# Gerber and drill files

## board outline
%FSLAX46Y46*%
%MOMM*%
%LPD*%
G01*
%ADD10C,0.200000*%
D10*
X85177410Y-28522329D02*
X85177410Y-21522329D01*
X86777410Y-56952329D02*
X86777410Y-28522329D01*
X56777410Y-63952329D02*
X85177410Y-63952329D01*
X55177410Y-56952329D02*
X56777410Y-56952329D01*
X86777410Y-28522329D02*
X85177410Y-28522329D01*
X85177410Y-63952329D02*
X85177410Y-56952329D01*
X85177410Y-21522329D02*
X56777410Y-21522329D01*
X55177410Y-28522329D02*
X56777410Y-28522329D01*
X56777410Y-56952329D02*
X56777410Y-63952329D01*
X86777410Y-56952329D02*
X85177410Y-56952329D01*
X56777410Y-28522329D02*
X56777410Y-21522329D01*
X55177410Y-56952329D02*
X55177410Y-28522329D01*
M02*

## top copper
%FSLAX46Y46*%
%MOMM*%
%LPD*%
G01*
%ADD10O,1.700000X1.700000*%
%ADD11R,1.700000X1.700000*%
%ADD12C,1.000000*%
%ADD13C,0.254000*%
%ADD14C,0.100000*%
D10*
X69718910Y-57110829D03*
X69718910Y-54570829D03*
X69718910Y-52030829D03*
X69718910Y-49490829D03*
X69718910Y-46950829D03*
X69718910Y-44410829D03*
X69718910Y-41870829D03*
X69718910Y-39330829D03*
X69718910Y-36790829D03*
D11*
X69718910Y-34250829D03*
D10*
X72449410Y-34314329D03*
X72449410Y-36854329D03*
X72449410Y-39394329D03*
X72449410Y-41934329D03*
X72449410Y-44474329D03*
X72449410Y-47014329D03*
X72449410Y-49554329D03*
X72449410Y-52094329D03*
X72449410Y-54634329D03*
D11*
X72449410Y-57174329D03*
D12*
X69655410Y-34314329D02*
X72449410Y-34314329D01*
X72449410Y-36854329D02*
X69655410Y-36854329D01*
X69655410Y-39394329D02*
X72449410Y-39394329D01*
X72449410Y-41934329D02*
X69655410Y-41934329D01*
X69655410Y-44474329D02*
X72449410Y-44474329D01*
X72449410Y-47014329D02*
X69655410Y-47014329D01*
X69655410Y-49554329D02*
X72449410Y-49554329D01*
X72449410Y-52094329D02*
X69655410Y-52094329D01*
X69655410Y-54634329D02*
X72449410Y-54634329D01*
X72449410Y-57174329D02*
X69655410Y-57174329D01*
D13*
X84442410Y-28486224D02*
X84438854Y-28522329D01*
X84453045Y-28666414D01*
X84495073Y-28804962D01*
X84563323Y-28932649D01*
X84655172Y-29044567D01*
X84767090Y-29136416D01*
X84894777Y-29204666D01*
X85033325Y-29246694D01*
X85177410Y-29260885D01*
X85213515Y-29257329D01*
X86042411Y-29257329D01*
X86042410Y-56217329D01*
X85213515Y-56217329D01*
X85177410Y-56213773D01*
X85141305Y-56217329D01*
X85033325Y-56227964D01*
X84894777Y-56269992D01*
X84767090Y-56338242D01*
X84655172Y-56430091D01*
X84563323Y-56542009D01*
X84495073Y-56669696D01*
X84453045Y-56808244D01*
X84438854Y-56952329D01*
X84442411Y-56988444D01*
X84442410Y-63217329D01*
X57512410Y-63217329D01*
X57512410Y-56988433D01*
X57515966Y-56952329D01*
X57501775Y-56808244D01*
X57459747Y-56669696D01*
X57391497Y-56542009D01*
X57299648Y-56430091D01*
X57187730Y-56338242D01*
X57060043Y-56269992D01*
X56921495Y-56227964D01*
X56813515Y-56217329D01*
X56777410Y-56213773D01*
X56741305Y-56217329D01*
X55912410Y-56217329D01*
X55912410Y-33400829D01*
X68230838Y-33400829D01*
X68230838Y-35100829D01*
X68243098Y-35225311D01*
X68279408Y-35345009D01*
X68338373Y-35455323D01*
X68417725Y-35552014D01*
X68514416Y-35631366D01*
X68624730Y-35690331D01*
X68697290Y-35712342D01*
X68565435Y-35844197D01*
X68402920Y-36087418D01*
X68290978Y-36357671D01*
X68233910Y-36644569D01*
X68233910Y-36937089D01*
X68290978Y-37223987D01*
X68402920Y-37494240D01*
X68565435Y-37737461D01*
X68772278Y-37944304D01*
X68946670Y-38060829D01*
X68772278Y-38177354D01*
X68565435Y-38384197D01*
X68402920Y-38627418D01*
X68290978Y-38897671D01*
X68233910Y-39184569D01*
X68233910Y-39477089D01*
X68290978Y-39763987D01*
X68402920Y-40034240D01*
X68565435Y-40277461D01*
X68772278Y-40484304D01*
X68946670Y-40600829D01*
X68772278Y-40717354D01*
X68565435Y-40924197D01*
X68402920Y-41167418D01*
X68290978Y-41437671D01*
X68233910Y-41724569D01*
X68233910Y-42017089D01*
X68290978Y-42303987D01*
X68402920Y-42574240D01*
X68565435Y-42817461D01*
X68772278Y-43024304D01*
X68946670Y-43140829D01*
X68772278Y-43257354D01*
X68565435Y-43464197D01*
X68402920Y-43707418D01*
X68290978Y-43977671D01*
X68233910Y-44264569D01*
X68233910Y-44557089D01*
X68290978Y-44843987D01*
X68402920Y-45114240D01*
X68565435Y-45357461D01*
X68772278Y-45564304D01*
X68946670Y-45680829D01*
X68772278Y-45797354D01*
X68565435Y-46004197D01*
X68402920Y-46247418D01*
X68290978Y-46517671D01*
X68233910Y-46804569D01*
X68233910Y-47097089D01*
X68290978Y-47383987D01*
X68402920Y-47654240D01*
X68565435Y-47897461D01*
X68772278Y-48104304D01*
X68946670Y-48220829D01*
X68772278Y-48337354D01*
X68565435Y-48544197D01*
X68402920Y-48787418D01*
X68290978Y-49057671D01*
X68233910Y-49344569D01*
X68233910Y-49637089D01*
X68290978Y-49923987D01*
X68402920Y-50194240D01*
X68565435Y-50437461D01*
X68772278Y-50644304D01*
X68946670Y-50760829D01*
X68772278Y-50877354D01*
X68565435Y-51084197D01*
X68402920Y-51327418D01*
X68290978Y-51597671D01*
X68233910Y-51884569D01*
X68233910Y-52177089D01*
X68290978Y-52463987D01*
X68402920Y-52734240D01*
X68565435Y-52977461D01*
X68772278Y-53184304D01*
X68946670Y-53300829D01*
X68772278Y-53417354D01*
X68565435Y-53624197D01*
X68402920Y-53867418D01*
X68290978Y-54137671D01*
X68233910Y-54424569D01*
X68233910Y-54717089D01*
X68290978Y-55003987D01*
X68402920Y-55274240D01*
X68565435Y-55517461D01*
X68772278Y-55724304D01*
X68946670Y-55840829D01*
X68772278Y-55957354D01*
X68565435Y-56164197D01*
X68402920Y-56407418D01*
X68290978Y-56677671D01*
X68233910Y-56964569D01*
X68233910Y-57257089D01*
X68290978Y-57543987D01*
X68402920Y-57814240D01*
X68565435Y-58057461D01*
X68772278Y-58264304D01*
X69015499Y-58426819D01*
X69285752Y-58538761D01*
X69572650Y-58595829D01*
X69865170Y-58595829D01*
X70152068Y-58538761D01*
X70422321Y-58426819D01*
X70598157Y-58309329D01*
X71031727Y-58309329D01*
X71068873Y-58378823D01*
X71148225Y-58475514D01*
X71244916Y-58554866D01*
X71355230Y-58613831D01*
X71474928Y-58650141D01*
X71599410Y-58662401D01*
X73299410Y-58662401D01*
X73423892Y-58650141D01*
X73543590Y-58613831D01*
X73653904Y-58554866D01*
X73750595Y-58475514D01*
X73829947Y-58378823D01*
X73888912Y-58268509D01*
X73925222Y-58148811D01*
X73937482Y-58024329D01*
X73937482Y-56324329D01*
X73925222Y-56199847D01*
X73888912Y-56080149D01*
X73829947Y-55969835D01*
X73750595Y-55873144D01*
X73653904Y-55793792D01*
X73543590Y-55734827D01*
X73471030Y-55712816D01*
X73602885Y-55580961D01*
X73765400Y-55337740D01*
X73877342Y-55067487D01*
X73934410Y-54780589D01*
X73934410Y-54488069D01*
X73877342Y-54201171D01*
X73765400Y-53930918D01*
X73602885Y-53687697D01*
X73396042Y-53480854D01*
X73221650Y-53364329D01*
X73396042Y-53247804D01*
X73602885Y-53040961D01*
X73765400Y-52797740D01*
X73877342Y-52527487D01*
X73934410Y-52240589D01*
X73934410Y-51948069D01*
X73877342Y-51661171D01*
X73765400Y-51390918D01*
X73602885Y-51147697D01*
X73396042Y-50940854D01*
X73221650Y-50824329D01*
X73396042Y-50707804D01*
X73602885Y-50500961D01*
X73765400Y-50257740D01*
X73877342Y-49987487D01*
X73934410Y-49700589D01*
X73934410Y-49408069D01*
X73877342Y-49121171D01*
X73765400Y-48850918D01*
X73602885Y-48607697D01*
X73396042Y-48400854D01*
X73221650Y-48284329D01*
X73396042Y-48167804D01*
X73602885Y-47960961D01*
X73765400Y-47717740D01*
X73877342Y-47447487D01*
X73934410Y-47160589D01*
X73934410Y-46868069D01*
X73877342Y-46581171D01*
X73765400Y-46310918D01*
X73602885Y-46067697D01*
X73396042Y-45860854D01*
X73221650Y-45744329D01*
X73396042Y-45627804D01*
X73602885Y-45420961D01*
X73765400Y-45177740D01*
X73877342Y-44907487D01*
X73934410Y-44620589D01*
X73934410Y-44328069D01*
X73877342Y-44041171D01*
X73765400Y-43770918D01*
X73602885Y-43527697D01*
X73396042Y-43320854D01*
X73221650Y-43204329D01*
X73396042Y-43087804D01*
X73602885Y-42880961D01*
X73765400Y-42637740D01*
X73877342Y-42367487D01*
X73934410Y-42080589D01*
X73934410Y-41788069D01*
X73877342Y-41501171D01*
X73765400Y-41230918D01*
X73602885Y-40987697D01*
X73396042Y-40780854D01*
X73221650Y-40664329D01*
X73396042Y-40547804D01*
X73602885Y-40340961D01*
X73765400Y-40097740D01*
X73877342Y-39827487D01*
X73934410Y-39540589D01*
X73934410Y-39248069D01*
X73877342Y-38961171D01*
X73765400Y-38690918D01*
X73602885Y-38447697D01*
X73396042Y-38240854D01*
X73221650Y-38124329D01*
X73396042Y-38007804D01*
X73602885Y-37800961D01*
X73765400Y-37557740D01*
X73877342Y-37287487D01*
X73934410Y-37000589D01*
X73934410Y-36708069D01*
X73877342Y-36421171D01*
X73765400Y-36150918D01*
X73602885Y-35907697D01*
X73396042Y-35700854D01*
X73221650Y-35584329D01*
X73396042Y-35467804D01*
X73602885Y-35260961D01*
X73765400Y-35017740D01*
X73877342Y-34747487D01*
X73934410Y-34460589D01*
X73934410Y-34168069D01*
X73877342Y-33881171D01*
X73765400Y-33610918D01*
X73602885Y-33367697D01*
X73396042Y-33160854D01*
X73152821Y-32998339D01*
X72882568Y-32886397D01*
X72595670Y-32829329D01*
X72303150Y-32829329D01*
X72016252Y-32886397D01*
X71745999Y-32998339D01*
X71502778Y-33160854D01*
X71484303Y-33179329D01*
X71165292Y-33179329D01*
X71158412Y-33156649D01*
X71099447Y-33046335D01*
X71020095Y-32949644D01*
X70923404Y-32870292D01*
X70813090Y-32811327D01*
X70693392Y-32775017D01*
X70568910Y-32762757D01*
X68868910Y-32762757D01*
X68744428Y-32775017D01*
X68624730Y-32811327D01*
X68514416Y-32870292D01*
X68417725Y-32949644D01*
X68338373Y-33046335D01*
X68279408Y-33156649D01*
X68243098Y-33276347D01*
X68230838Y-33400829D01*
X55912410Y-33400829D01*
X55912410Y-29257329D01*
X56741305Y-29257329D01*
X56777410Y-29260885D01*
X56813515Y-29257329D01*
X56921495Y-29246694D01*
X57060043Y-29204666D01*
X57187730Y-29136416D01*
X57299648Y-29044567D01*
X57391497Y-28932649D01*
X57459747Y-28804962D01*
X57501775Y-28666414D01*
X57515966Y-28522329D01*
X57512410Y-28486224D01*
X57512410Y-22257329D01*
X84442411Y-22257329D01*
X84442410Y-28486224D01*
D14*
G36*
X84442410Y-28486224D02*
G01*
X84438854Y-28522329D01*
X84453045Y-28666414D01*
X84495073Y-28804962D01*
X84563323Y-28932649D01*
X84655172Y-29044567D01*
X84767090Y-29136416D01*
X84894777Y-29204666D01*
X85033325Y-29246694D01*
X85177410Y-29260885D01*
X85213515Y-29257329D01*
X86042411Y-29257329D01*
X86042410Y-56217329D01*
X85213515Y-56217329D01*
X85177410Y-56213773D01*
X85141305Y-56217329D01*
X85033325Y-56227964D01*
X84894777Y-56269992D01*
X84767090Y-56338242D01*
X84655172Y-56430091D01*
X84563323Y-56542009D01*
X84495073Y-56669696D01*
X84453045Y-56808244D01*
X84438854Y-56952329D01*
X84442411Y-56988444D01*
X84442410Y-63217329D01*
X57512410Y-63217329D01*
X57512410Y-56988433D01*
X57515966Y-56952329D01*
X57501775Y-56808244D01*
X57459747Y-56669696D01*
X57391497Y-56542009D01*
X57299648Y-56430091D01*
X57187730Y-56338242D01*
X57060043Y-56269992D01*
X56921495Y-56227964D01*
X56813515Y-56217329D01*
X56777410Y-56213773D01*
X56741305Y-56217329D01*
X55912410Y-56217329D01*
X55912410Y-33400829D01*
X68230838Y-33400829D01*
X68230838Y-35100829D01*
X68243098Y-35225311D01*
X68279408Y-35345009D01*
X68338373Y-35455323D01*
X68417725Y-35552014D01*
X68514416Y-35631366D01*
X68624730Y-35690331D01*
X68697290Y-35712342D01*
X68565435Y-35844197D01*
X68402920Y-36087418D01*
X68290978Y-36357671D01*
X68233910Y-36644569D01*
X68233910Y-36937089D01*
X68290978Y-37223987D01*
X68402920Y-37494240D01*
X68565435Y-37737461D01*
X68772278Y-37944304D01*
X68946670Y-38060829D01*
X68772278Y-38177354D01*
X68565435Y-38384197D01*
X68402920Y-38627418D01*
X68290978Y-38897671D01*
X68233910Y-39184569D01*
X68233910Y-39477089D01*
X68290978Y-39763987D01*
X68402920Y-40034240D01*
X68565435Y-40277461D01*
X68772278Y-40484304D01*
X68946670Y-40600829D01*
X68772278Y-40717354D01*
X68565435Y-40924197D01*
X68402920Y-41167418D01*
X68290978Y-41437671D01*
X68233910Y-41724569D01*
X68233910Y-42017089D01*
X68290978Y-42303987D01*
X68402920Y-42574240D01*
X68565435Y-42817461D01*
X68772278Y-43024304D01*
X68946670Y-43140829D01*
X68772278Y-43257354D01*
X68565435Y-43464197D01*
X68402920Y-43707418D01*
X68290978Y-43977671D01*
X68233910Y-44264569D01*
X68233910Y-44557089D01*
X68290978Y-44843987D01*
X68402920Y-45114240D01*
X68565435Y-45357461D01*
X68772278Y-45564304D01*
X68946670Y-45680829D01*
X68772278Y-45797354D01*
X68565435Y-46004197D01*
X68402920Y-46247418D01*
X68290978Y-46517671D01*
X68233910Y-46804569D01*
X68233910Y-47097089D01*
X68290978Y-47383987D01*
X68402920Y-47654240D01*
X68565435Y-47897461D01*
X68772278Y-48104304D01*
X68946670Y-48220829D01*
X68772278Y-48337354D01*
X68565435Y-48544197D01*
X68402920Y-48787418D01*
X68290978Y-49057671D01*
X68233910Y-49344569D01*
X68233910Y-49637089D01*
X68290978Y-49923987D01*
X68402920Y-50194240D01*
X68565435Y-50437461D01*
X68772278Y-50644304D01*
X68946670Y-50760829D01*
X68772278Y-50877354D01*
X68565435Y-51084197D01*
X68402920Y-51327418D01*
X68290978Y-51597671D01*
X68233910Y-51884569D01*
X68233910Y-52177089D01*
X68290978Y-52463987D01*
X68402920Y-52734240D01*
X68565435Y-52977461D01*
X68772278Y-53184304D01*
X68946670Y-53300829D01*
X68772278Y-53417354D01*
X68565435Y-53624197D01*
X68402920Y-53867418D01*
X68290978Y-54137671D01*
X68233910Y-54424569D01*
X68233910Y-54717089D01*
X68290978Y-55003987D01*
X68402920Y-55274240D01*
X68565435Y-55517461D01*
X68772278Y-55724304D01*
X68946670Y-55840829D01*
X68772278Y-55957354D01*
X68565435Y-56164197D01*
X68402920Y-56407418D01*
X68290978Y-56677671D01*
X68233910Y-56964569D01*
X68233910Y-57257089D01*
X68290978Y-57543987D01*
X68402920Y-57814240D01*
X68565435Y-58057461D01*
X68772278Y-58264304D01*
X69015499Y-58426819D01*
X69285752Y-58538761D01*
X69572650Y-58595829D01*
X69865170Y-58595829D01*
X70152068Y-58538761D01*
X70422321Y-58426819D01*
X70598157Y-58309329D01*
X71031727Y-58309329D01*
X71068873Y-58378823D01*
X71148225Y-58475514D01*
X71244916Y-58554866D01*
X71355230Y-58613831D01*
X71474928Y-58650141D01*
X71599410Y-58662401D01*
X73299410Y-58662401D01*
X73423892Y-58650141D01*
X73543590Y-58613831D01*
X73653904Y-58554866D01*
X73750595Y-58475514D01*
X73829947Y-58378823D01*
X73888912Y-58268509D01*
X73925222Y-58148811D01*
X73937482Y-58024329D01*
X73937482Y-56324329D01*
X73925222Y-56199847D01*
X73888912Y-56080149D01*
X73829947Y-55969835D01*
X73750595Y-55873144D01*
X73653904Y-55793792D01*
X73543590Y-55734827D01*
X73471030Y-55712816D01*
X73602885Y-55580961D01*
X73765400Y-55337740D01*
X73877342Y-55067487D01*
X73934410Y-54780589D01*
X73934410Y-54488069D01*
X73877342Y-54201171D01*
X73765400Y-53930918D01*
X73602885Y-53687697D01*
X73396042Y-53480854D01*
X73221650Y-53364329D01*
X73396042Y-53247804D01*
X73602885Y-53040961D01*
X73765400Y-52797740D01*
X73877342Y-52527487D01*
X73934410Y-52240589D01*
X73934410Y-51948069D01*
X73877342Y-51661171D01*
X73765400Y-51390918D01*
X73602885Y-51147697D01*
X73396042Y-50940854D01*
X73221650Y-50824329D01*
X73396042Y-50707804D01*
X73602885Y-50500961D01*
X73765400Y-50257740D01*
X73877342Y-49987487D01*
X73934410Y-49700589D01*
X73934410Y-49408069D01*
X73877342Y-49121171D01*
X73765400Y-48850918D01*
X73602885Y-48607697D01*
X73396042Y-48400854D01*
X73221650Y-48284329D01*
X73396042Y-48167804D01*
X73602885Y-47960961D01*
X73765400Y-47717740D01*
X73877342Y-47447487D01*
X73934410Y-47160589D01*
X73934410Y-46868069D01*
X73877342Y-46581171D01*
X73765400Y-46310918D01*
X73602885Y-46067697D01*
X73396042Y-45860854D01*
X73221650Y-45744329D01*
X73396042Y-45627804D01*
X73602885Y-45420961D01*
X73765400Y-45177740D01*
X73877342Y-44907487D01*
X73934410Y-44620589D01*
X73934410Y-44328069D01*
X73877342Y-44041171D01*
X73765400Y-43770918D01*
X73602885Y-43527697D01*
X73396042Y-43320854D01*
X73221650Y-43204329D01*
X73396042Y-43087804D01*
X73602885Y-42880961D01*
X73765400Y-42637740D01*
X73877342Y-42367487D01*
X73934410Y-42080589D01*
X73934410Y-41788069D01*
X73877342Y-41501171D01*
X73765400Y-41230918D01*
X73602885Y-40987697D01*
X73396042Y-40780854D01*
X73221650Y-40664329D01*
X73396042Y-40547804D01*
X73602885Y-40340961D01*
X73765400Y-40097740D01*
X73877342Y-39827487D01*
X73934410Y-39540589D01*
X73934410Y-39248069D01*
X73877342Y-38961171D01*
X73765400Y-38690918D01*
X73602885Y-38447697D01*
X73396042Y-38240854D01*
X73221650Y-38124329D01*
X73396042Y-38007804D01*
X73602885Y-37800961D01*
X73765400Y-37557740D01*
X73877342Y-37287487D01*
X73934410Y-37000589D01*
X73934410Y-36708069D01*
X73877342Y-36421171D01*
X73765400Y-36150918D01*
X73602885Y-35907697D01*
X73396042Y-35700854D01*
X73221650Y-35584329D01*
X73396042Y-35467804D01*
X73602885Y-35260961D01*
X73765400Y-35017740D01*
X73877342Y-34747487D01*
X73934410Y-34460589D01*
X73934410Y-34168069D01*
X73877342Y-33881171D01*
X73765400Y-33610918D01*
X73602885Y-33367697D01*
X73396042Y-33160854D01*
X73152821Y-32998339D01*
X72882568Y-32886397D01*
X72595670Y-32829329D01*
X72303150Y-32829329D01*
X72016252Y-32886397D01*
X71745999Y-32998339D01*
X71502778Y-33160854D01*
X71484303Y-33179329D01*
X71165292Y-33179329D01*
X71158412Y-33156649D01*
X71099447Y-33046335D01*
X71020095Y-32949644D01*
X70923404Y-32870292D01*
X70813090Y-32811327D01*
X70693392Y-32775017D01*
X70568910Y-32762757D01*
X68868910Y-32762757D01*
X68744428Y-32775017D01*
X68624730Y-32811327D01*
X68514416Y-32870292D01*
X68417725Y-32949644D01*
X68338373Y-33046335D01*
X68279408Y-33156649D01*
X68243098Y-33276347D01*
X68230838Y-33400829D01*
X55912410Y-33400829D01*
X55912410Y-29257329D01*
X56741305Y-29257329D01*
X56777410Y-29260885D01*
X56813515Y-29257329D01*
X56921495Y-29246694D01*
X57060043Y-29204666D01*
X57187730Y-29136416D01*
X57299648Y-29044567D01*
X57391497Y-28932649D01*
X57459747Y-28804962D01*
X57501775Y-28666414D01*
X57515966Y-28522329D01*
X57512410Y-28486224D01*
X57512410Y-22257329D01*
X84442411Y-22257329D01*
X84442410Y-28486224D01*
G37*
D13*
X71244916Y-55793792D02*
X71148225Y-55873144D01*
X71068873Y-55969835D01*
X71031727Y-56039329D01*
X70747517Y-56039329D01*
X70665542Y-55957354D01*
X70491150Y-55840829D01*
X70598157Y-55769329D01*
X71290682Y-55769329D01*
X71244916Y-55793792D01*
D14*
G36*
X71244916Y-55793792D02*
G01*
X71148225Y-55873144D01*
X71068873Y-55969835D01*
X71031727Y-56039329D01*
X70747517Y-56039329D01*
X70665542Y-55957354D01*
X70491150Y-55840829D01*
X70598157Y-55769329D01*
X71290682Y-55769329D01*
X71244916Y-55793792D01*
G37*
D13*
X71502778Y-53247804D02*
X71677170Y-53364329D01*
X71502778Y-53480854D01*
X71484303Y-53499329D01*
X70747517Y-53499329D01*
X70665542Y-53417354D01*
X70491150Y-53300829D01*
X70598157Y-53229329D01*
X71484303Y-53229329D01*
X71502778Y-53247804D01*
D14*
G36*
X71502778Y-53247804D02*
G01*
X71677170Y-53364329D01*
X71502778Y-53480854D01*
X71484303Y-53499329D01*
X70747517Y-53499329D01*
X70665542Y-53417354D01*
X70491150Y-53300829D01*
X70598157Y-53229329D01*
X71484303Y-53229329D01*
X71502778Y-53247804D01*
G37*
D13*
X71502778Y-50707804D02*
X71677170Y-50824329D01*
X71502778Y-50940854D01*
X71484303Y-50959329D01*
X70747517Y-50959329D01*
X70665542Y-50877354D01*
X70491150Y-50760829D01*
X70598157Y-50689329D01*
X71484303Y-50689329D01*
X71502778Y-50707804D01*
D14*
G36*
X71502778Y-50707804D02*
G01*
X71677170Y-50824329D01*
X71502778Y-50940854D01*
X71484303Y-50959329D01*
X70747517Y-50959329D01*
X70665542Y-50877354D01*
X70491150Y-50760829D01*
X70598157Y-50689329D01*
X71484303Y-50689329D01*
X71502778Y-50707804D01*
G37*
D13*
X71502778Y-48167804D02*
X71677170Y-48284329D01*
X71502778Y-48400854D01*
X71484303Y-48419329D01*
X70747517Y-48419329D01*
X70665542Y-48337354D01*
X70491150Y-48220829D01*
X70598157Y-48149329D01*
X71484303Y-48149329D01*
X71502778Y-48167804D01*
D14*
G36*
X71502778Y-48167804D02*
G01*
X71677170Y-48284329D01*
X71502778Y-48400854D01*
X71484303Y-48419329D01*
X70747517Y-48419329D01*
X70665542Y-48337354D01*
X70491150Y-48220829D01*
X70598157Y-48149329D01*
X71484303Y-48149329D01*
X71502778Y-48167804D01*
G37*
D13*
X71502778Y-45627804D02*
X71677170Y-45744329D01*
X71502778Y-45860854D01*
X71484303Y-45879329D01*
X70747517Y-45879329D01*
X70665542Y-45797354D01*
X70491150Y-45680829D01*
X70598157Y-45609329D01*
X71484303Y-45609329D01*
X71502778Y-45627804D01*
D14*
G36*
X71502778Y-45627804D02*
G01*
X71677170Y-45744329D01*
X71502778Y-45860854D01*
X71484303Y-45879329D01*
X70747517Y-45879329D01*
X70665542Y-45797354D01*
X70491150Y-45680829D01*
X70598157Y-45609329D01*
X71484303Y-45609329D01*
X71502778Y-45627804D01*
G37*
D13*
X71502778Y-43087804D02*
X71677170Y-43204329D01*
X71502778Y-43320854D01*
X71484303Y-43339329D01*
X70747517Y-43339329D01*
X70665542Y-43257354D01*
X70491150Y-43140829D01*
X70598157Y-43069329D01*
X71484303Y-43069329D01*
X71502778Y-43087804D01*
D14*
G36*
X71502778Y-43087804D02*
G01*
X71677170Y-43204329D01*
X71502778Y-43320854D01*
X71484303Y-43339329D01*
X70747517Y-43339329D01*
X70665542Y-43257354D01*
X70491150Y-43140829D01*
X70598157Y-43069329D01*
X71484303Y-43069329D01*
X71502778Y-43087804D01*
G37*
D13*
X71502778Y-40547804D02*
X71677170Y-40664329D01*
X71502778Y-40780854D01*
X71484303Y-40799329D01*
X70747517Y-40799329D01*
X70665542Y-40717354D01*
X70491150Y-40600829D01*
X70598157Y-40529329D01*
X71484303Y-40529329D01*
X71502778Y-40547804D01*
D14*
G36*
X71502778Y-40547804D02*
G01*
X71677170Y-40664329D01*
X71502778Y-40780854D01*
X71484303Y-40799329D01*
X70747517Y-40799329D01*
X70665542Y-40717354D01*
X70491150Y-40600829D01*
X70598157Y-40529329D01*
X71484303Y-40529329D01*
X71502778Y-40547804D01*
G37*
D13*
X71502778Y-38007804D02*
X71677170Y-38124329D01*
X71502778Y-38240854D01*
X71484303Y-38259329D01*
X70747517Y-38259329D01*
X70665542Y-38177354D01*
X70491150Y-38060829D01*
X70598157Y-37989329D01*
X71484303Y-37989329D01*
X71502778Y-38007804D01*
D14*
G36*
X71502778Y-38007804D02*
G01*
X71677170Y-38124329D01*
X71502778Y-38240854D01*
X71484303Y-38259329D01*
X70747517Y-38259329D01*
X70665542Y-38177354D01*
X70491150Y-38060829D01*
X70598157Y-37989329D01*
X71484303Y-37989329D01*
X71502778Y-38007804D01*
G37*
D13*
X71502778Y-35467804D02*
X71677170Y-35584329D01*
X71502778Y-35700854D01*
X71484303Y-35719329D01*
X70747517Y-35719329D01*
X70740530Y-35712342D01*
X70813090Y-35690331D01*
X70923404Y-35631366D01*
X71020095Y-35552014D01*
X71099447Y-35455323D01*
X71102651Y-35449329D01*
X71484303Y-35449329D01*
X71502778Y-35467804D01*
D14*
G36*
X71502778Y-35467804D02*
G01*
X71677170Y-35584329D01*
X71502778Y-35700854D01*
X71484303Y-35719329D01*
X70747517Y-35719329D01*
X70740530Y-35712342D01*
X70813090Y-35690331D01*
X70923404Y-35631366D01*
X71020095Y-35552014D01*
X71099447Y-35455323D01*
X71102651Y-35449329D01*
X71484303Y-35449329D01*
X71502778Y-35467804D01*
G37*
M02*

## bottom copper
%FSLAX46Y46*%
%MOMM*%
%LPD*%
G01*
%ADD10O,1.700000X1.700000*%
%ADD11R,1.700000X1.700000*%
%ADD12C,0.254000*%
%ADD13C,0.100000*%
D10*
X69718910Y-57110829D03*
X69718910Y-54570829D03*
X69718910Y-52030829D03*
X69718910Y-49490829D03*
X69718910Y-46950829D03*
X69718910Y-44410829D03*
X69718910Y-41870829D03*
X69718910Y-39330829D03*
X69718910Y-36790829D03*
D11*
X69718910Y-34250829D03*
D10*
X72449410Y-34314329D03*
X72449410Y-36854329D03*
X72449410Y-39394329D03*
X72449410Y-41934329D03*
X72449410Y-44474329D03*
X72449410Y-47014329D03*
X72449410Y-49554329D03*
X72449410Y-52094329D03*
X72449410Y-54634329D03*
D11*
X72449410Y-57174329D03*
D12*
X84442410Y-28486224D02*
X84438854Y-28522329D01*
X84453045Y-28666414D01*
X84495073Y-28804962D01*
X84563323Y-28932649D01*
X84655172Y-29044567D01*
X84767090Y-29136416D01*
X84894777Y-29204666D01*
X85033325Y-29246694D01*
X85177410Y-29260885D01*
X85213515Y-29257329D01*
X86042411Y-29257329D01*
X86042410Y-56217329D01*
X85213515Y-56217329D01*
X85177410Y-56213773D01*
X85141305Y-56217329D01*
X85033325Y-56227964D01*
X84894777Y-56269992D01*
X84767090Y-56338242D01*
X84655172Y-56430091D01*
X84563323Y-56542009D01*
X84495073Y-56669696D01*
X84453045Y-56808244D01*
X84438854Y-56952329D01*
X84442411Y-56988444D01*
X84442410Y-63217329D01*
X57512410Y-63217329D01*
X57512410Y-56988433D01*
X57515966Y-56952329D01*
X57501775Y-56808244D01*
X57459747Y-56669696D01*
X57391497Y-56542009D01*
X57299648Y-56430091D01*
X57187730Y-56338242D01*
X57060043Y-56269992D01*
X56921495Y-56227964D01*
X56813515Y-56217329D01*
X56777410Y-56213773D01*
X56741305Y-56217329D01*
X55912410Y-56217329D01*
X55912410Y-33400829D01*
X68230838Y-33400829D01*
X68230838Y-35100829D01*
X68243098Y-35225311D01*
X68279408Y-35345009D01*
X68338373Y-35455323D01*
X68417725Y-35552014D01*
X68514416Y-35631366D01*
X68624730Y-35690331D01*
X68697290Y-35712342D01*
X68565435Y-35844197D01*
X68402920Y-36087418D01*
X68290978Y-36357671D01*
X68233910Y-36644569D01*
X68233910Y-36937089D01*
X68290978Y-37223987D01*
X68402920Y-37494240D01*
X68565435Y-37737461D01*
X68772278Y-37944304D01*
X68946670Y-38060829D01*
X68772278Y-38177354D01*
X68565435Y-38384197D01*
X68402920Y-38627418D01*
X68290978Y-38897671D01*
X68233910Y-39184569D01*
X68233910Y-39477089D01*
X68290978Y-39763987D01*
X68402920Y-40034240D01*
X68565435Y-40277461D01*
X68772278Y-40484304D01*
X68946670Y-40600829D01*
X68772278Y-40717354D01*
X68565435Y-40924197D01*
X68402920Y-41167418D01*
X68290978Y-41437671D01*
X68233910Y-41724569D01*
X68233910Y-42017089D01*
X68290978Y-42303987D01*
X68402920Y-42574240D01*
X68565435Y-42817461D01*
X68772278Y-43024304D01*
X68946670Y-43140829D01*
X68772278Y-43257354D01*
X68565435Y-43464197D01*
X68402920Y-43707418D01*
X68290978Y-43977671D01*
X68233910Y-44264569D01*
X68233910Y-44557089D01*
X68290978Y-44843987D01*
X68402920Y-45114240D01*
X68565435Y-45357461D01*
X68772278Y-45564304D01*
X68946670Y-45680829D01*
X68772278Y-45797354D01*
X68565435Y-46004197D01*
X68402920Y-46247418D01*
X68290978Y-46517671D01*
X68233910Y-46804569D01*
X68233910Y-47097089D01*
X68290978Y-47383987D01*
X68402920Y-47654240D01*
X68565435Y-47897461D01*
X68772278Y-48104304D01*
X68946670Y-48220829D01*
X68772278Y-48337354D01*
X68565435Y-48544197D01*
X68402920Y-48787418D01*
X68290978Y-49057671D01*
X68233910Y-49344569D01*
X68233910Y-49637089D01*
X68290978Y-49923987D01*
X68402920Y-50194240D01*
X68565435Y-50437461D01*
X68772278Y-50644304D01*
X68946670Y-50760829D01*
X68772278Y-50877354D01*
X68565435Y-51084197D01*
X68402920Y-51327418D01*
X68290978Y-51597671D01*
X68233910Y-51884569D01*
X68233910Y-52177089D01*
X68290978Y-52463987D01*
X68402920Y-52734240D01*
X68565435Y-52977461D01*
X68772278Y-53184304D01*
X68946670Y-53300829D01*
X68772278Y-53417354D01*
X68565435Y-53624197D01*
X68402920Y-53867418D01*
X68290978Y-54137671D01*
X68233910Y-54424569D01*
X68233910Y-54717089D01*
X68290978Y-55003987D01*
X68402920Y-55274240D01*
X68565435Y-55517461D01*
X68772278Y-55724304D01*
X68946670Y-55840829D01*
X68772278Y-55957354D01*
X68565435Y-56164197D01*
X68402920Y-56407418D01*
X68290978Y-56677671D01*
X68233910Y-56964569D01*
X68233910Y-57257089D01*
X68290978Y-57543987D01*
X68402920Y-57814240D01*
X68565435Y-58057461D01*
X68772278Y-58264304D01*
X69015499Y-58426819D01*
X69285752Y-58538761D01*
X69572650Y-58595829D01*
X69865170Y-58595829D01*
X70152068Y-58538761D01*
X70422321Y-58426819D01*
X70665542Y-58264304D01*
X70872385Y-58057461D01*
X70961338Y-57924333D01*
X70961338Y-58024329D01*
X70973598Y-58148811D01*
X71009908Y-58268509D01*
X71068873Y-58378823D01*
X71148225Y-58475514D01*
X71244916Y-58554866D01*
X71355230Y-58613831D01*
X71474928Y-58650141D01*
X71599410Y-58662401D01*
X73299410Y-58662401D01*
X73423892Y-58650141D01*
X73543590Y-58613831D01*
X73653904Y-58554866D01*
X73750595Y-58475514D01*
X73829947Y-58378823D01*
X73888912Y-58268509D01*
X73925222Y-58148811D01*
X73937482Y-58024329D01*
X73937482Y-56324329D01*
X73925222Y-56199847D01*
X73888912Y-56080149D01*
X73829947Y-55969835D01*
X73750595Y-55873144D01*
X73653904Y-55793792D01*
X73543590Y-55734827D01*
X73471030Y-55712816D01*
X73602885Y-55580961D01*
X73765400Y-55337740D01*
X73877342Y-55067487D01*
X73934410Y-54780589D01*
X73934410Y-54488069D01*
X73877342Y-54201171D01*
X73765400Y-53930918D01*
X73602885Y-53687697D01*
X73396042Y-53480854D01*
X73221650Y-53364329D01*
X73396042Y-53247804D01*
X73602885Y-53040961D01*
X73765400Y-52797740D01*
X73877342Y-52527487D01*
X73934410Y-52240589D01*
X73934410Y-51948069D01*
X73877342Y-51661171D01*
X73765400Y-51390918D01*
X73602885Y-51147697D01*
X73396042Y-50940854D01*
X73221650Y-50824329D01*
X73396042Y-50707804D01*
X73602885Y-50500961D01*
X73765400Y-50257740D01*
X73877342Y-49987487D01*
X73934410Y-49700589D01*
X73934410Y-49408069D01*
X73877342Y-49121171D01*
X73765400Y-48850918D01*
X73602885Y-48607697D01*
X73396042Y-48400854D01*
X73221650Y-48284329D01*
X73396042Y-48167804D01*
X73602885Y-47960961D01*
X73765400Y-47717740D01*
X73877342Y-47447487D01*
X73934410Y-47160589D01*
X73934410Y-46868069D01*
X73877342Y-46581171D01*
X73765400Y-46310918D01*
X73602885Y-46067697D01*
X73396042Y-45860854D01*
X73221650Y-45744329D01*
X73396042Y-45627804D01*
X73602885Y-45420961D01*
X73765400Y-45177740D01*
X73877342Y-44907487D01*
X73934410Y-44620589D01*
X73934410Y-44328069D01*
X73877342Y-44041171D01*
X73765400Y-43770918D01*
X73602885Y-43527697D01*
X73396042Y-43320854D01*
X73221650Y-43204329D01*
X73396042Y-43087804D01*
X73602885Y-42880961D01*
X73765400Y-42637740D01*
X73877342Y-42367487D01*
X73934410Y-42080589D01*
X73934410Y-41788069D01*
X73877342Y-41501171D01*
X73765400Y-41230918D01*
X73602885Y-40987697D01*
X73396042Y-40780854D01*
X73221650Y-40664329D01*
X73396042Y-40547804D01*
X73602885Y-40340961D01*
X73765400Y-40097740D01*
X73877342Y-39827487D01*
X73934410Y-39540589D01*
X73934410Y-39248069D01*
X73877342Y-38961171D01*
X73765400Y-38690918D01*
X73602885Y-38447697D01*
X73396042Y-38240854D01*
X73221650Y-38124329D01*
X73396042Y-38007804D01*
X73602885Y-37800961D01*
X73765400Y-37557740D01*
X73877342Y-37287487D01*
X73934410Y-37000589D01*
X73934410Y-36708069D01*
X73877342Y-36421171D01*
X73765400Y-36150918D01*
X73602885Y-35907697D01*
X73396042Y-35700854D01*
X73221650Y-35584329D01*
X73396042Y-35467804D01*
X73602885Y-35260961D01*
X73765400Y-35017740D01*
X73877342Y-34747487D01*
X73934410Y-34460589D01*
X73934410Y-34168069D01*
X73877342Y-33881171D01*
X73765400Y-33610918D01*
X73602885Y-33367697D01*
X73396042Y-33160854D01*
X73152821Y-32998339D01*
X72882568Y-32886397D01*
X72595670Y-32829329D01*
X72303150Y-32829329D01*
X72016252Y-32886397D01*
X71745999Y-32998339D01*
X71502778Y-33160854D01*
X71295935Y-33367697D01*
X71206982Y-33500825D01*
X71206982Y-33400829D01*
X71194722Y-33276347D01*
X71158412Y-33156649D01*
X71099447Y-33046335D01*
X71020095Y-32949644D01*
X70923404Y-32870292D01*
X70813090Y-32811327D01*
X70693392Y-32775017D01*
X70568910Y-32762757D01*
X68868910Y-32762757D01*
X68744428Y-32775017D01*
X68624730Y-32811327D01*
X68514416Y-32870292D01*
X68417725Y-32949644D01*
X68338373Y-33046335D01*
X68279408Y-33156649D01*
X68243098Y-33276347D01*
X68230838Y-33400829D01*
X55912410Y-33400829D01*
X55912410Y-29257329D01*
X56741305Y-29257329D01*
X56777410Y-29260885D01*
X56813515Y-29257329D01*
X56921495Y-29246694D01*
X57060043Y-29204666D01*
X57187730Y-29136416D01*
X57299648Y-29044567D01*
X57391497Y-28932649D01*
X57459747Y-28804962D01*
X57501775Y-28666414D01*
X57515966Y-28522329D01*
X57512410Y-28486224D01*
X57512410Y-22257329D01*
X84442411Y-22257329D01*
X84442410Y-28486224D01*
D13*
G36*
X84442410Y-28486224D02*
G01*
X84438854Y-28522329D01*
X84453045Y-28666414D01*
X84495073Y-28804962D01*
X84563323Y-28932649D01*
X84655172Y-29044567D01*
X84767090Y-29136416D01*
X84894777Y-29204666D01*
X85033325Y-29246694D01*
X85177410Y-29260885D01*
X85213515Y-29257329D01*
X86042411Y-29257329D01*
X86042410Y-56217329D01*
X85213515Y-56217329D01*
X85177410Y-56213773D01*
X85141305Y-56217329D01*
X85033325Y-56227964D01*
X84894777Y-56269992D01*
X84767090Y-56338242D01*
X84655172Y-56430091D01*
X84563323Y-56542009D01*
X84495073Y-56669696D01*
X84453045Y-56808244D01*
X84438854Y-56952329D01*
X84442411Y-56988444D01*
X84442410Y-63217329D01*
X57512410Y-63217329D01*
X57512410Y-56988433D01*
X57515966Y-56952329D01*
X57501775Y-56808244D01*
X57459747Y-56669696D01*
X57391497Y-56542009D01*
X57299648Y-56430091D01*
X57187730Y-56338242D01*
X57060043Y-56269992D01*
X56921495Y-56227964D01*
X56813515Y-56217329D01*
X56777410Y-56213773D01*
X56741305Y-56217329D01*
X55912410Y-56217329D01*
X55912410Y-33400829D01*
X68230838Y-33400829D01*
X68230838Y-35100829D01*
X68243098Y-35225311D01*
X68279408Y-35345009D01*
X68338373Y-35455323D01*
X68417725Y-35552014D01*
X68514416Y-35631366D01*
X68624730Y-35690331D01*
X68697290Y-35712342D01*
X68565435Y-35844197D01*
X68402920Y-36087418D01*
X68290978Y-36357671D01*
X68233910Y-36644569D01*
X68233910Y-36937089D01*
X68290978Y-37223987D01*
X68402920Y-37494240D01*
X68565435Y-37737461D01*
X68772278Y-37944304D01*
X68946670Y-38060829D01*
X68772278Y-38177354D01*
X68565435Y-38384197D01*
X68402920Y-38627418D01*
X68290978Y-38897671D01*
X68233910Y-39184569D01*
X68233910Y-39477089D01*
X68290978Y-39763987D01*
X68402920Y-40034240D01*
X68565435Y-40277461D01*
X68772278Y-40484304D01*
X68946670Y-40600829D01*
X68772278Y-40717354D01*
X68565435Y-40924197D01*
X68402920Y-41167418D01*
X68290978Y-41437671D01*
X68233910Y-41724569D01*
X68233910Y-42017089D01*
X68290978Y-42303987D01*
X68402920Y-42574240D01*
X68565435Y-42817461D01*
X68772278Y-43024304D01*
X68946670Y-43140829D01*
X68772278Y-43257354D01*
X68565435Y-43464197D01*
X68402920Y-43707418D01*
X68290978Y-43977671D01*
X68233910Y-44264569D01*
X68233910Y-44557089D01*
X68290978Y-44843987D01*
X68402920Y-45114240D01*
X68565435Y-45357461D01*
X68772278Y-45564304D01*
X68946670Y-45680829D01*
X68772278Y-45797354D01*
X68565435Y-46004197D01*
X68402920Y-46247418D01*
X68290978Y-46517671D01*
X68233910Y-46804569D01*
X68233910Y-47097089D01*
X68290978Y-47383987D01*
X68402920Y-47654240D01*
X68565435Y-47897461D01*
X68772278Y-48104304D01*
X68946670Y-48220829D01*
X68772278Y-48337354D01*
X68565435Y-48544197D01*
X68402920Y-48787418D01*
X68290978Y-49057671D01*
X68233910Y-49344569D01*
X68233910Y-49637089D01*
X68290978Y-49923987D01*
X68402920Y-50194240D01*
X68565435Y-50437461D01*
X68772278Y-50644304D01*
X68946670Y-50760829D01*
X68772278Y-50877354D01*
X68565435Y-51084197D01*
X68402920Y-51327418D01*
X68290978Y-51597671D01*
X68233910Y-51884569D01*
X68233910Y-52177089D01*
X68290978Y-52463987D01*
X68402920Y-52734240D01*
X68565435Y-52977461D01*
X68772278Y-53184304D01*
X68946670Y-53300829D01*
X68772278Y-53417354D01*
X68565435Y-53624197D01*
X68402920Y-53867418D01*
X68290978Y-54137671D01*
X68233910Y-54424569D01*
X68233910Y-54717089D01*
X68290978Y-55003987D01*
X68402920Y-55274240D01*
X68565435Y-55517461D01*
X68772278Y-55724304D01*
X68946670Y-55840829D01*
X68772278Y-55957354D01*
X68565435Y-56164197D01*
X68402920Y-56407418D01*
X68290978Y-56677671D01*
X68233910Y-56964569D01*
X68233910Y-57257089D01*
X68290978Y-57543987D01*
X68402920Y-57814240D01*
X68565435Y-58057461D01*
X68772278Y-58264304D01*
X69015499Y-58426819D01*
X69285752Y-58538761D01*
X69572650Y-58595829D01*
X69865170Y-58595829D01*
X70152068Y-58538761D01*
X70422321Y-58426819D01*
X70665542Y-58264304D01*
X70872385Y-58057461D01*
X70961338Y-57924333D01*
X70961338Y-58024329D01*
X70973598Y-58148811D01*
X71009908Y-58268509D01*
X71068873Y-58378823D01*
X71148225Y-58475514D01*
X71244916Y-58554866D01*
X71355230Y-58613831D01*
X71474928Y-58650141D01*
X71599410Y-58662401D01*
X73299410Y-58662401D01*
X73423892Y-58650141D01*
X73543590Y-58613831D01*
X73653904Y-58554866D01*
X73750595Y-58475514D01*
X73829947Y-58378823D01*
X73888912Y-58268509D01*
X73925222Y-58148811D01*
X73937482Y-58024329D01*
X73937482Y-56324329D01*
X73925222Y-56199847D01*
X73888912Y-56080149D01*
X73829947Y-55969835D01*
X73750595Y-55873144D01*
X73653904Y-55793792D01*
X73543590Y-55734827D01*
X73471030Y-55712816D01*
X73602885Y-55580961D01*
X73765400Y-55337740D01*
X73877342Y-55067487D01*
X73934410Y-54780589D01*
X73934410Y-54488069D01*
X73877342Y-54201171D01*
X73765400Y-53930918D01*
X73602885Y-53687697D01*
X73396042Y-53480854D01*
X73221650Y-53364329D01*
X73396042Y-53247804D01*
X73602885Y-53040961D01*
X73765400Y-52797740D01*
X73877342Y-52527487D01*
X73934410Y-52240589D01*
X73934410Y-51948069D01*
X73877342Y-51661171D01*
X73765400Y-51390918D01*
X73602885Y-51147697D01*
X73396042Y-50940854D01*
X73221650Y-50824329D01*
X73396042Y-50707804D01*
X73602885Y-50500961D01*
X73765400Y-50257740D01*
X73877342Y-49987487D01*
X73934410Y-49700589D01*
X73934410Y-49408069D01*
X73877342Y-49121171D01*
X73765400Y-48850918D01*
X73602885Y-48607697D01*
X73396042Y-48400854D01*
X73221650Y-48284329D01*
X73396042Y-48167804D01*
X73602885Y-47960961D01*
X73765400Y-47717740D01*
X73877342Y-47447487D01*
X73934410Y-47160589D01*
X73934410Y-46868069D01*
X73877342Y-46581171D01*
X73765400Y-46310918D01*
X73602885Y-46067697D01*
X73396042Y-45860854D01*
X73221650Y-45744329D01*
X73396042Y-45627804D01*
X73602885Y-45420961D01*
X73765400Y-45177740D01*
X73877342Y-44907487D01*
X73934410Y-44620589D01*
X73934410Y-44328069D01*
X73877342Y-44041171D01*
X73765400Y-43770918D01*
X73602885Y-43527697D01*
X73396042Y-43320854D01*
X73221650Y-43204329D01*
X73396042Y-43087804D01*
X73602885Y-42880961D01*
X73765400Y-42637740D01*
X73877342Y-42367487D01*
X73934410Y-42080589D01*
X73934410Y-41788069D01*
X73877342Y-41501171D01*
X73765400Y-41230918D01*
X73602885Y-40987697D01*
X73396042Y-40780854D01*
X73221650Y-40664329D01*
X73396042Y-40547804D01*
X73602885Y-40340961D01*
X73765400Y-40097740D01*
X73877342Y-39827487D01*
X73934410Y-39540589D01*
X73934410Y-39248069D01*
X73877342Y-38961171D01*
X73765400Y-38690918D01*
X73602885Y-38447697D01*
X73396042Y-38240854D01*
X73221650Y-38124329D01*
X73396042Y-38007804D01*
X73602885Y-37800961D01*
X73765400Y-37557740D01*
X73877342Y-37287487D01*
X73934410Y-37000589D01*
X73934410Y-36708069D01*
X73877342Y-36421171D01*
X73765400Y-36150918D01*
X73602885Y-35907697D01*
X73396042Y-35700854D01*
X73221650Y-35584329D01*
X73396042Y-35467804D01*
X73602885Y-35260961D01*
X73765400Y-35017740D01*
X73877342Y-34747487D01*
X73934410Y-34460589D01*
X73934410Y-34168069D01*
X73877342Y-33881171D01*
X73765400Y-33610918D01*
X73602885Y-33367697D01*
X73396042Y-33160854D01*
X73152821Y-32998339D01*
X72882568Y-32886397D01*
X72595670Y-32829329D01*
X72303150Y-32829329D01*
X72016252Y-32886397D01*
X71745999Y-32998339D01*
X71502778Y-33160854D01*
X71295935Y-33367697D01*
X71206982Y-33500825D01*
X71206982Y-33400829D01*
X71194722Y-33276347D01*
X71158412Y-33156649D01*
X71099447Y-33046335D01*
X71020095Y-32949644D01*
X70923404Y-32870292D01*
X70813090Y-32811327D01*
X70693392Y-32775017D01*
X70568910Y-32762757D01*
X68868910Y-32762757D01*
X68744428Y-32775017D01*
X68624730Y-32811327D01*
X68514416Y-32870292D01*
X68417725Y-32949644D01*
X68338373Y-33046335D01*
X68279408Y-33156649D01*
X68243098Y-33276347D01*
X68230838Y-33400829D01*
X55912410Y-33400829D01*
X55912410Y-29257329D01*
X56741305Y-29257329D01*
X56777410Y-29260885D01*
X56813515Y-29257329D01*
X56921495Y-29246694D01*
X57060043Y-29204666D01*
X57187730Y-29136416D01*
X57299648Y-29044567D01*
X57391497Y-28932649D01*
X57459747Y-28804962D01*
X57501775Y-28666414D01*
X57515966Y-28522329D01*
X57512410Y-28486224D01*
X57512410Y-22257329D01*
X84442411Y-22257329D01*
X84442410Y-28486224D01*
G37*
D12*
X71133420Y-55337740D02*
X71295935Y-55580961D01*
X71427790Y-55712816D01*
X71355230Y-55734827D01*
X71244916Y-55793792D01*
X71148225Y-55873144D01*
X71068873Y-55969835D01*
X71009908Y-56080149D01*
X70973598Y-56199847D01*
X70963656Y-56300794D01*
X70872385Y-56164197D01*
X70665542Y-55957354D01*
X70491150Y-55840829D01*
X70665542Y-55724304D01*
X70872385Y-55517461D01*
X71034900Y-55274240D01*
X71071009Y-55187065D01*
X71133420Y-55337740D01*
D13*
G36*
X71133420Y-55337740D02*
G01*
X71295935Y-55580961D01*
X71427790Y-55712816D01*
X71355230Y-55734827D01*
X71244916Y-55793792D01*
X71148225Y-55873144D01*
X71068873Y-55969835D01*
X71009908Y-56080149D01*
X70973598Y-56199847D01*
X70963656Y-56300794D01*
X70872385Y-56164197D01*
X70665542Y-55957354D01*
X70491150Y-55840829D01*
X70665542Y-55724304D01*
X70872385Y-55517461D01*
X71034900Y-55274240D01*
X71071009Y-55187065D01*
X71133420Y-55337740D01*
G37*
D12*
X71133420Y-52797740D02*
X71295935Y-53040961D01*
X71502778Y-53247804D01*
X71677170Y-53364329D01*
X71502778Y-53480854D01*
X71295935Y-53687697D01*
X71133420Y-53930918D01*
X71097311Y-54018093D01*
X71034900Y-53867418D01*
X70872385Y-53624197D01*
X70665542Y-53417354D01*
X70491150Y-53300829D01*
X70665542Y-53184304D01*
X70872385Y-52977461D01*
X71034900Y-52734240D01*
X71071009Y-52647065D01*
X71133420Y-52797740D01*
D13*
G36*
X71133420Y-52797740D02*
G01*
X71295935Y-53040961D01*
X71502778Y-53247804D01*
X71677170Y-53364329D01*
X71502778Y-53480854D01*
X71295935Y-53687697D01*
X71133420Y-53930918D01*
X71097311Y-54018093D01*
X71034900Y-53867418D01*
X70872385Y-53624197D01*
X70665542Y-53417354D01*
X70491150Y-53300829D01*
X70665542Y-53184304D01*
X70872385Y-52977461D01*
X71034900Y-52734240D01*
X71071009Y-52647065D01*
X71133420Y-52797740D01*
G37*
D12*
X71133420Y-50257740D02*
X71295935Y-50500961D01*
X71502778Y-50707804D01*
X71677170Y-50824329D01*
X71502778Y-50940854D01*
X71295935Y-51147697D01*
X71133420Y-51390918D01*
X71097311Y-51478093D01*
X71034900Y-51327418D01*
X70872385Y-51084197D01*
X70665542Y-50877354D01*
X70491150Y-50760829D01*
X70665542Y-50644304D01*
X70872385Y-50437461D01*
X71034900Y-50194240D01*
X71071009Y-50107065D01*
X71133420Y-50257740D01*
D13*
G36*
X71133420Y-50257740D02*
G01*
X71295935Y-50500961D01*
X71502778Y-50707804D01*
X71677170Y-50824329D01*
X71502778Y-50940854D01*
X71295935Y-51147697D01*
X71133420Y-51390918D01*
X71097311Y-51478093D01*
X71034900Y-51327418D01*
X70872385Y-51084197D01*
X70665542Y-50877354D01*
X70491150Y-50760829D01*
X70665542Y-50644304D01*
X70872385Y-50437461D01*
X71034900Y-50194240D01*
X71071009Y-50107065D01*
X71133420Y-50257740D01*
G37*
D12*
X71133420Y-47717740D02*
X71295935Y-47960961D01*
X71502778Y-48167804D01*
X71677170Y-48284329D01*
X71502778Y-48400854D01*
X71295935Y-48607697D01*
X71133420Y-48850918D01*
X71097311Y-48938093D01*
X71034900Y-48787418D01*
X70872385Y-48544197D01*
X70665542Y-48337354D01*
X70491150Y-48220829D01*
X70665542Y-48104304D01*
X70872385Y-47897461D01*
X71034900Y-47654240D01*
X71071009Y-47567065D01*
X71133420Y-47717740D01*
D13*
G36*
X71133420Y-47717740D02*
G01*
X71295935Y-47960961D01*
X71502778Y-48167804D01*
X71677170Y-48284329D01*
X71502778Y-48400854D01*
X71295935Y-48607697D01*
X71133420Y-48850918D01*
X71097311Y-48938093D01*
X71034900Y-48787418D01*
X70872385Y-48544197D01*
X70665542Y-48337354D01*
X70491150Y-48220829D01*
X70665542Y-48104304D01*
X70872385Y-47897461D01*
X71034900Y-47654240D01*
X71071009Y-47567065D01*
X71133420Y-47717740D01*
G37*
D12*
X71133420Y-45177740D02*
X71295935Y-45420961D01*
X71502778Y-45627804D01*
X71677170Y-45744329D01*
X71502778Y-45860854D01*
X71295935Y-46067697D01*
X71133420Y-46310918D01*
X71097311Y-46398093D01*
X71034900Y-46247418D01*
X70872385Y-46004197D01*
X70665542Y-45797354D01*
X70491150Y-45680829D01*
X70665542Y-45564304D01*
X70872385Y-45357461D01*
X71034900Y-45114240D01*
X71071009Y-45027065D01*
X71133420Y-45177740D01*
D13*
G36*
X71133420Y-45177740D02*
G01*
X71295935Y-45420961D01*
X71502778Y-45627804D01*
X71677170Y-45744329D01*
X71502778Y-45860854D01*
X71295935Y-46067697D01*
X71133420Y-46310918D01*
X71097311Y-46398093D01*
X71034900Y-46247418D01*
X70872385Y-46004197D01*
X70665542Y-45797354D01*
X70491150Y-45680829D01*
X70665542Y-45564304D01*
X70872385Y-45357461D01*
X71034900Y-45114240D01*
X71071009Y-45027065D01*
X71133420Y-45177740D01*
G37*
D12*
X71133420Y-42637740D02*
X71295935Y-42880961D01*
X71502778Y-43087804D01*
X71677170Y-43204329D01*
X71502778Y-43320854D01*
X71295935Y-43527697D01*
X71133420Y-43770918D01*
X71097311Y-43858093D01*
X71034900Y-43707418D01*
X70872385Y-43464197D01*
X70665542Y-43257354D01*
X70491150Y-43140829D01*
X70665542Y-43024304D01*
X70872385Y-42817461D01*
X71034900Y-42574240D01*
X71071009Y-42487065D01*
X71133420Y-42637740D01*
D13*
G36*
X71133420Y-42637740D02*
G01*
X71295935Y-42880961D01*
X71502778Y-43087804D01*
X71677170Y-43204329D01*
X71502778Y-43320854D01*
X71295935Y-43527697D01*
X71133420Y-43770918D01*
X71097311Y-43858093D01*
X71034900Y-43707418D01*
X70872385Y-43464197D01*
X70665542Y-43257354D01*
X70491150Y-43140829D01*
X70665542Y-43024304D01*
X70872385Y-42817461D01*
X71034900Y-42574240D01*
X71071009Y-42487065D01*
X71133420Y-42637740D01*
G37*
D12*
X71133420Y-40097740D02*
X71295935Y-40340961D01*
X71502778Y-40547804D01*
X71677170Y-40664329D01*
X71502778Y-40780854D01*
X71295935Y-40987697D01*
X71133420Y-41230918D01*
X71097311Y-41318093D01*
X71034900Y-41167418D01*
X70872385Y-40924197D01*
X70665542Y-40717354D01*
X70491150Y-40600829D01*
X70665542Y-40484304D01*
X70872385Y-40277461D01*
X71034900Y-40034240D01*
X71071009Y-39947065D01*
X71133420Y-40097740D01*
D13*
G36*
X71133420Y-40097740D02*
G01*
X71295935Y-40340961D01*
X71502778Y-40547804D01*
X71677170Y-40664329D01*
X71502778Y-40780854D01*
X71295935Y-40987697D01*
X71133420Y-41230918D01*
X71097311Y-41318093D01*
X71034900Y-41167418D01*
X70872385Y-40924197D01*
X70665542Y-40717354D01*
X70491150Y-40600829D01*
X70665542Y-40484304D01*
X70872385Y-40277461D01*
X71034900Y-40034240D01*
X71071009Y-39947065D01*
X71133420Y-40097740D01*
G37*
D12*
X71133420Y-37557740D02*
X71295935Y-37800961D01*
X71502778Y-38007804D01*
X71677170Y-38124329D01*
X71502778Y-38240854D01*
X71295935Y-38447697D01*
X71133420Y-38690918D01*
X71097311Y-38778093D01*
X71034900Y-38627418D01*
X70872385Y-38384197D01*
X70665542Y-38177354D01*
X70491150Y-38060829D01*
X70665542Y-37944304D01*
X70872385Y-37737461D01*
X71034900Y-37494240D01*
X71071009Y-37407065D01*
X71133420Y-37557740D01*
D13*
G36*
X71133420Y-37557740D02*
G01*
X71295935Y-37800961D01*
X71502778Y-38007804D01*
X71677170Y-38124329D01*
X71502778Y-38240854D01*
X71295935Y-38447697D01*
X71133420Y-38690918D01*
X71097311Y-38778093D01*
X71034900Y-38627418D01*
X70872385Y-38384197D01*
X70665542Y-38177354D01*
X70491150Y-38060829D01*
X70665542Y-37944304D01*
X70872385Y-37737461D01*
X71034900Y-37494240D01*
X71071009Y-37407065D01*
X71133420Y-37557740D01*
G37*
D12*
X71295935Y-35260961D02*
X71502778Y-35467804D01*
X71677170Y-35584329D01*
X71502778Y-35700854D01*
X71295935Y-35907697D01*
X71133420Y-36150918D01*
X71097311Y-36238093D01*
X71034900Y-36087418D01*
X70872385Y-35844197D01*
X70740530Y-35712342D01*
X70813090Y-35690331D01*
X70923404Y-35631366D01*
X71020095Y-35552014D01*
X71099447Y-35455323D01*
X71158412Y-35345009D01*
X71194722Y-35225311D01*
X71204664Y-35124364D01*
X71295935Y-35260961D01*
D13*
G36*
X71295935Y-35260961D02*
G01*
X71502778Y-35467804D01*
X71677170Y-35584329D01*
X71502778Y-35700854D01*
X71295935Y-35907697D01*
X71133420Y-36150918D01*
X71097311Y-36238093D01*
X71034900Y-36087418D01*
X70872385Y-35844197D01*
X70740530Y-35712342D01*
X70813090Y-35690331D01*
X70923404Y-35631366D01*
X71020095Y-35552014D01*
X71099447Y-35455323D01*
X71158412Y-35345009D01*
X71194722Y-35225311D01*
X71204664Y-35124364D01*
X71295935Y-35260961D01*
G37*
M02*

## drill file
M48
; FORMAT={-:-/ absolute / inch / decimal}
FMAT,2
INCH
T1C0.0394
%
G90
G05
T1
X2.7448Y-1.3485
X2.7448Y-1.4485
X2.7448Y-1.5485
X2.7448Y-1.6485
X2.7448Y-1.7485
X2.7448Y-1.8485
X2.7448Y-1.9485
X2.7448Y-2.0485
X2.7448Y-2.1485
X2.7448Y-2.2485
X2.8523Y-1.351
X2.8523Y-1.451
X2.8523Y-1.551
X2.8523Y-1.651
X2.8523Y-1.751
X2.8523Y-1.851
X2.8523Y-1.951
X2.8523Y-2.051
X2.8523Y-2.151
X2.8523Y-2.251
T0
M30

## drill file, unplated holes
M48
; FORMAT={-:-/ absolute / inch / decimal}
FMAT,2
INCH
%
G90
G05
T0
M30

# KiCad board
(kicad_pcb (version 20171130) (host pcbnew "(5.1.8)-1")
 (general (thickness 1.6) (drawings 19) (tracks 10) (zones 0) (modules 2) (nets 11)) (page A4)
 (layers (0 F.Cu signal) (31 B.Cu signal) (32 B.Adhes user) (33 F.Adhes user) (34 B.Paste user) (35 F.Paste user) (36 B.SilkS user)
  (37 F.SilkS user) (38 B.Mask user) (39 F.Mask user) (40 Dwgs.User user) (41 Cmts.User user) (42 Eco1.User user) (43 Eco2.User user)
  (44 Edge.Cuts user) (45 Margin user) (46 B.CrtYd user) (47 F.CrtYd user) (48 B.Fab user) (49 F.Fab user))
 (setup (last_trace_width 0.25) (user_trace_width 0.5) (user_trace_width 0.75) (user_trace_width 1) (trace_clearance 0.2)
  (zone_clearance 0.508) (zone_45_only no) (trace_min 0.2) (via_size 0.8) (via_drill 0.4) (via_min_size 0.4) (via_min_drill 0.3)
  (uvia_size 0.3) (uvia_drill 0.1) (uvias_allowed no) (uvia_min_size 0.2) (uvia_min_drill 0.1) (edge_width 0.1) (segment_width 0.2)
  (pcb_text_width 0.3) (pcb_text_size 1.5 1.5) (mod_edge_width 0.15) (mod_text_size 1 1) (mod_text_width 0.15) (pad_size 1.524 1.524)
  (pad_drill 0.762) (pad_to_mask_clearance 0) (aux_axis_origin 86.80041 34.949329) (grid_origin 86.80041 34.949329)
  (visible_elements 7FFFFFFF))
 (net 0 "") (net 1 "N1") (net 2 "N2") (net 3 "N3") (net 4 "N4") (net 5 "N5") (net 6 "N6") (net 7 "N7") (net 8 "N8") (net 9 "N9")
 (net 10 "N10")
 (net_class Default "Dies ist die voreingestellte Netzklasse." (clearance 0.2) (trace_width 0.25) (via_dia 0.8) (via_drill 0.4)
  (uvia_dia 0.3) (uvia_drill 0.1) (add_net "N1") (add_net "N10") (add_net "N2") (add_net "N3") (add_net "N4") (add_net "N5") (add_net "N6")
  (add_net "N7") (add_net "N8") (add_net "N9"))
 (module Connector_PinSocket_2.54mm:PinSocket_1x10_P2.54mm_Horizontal (layer F.Cu) (at 69.71891 34.250829)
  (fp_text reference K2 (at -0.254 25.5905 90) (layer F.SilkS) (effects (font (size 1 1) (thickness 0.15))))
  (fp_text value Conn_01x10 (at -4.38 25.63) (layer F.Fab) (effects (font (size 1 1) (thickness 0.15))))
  (pad 10 thru_hole oval (at 0 22.86) (size 1.7 1.7) (drill 1) (layers *.Cu *.Mask) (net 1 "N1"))
  (pad 9 thru_hole oval (at 0 20.32) (size 1.7 1.7) (drill 1) (layers *.Cu *.Mask) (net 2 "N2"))
  (pad 8 thru_hole oval (at 0 17.78) (size 1.7 1.7) (drill 1) (layers *.Cu *.Mask) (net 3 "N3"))
  (pad 7 thru_hole oval (at 0 15.24) (size 1.7 1.7) (drill 1) (layers *.Cu *.Mask) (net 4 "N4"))
  (pad 6 thru_hole oval (at 0 12.7) (size 1.7 1.7) (drill 1) (layers *.Cu *.Mask) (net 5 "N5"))
  (pad 5 thru_hole oval (at 0 10.16) (size 1.7 1.7) (drill 1) (layers *.Cu *.Mask) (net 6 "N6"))
  (pad 4 thru_hole oval (at 0 7.62) (size 1.7 1.7) (drill 1) (layers *.Cu *.Mask) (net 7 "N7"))
  (pad 3 thru_hole oval (at 0 5.08) (size 1.7 1.7) (drill 1) (layers *.Cu *.Mask) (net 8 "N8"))
  (pad 2 thru_hole oval (at 0 2.54) (size 1.7 1.7) (drill 1) (layers *.Cu *.Mask) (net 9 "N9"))
  (pad 1 thru_hole rect (at 0 0) (size 1.7 1.7) (drill 1) (layers *.Cu *.Mask) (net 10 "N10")))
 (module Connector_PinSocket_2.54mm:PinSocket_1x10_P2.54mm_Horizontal (layer F.Cu) (at 72.44941 57.174329 180)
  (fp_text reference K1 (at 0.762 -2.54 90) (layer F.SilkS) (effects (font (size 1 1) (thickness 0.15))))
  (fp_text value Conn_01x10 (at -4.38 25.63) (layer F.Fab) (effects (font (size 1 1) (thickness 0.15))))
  (pad 10 thru_hole oval (at 0 22.86 180) (size 1.7 1.7) (drill 1) (layers *.Cu *.Mask) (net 10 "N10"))
  (pad 9 thru_hole oval (at 0 20.32 180) (size 1.7 1.7) (drill 1) (layers *.Cu *.Mask) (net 9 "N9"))
  (pad 8 thru_hole oval (at 0 17.78 180) (size 1.7 1.7) (drill 1) (layers *.Cu *.Mask) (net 8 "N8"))
  (pad 7 thru_hole oval (at 0 15.24 180) (size 1.7 1.7) (drill 1) (layers *.Cu *.Mask) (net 7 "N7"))
  (pad 6 thru_hole oval (at 0 12.7 180) (size 1.7 1.7) (drill 1) (layers *.Cu *.Mask) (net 6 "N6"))
  (pad 5 thru_hole oval (at 0 10.16 180) (size 1.7 1.7) (drill 1) (layers *.Cu *.Mask) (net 5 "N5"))
  (pad 4 thru_hole oval (at 0 7.62 180) (size 1.7 1.7) (drill 1) (layers *.Cu *.Mask) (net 4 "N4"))
  (pad 3 thru_hole oval (at 0 5.08 180) (size 1.7 1.7) (drill 1) (layers *.Cu *.Mask) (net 3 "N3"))
  (pad 2 thru_hole oval (at 0 2.54 180) (size 1.7 1.7) (drill 1) (layers *.Cu *.Mask) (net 2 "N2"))
  (pad 1 thru_hole rect (at 0 0 180) (size 1.7 1.7) (drill 1) (layers *.Cu *.Mask) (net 1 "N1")))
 (gr_line (start 85.17741 28.522329) (end 85.17741 21.522329) (layer Edge.Cuts) (width 0.2))
 (gr_line (start 86.77741 56.952329) (end 86.77741 28.522329) (layer Edge.Cuts) (width 0.2))
 (gr_line (start 56.77741 63.952329) (end 85.17741 63.952329) (layer Edge.Cuts) (width 0.2))
 (gr_line (start 55.17741 56.952329) (end 56.77741 56.952329) (layer Edge.Cuts) (width 0.2))
 (gr_line (start 86.77741 28.522329) (end 85.17741 28.522329) (layer Edge.Cuts) (width 0.2))
 (gr_line (start 85.17741 63.952329) (end 85.17741 56.952329) (layer Edge.Cuts) (width 0.2))
 (gr_line (start 85.17741 21.522329) (end 56.77741 21.522329) (layer Edge.Cuts) (width 0.2))
 (gr_line (start 55.17741 28.522329) (end 56.77741 28.522329) (layer Edge.Cuts) (width 0.2))
 (gr_line (start 56.77741 56.952329) (end 56.77741 63.952329) (layer Edge.Cuts) (width 0.2))
 (gr_line (start 86.77741 56.952329) (end 85.17741 56.952329) (layer Edge.Cuts) (width 0.2))
 (gr_line (start 56.77741 28.522329) (end 56.77741 21.522329) (layer Edge.Cuts) (width 0.2))
 (gr_line (start 55.17741 56.952329) (end 55.17741 28.522329) (layer Edge.Cuts) (width 0.2))
 (segment (start 69.65541 34.314329) (end 72.44941 34.314329) (width 1) (layer F.Cu) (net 10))
 (segment (start 72.44941 36.854329) (end 69.65541 36.854329) (width 1) (layer F.Cu) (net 9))
 (segment (start 69.65541 39.394329) (end 72.44941 39.394329) (width 1) (layer F.Cu) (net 8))
 (segment (start 72.44941 41.934329) (end 69.65541 41.934329) (width 1) (layer F.Cu) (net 7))
 (segment (start 69.65541 44.474329) (end 72.44941 44.474329) (width 1) (layer F.Cu) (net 6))
 (segment (start 72.44941 47.014329) (end 69.65541 47.014329) (width 1) (layer F.Cu) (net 5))
 (segment (start 69.65541 49.554329) (end 72.44941 49.554329) (width 1) (layer F.Cu) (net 4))
 (segment (start 72.44941 52.094329) (end 69.65541 52.094329) (width 1) (layer F.Cu) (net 3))
 (segment (start 69.65541 54.634329) (end 72.44941 54.634329) (width 1) (layer F.Cu) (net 2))
 (segment (start 72.44941 57.174329) (end 69.65541 57.174329) (width 1) (layer F.Cu) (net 1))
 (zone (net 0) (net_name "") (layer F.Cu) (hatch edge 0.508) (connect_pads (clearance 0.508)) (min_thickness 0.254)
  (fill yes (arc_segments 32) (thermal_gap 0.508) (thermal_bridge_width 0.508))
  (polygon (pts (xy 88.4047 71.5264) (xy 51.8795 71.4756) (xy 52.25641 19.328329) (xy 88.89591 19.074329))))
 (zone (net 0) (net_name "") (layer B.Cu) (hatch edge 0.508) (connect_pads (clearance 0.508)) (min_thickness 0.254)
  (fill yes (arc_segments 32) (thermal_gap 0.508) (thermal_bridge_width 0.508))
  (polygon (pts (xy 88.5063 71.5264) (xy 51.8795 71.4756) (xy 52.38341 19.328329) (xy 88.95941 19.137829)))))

